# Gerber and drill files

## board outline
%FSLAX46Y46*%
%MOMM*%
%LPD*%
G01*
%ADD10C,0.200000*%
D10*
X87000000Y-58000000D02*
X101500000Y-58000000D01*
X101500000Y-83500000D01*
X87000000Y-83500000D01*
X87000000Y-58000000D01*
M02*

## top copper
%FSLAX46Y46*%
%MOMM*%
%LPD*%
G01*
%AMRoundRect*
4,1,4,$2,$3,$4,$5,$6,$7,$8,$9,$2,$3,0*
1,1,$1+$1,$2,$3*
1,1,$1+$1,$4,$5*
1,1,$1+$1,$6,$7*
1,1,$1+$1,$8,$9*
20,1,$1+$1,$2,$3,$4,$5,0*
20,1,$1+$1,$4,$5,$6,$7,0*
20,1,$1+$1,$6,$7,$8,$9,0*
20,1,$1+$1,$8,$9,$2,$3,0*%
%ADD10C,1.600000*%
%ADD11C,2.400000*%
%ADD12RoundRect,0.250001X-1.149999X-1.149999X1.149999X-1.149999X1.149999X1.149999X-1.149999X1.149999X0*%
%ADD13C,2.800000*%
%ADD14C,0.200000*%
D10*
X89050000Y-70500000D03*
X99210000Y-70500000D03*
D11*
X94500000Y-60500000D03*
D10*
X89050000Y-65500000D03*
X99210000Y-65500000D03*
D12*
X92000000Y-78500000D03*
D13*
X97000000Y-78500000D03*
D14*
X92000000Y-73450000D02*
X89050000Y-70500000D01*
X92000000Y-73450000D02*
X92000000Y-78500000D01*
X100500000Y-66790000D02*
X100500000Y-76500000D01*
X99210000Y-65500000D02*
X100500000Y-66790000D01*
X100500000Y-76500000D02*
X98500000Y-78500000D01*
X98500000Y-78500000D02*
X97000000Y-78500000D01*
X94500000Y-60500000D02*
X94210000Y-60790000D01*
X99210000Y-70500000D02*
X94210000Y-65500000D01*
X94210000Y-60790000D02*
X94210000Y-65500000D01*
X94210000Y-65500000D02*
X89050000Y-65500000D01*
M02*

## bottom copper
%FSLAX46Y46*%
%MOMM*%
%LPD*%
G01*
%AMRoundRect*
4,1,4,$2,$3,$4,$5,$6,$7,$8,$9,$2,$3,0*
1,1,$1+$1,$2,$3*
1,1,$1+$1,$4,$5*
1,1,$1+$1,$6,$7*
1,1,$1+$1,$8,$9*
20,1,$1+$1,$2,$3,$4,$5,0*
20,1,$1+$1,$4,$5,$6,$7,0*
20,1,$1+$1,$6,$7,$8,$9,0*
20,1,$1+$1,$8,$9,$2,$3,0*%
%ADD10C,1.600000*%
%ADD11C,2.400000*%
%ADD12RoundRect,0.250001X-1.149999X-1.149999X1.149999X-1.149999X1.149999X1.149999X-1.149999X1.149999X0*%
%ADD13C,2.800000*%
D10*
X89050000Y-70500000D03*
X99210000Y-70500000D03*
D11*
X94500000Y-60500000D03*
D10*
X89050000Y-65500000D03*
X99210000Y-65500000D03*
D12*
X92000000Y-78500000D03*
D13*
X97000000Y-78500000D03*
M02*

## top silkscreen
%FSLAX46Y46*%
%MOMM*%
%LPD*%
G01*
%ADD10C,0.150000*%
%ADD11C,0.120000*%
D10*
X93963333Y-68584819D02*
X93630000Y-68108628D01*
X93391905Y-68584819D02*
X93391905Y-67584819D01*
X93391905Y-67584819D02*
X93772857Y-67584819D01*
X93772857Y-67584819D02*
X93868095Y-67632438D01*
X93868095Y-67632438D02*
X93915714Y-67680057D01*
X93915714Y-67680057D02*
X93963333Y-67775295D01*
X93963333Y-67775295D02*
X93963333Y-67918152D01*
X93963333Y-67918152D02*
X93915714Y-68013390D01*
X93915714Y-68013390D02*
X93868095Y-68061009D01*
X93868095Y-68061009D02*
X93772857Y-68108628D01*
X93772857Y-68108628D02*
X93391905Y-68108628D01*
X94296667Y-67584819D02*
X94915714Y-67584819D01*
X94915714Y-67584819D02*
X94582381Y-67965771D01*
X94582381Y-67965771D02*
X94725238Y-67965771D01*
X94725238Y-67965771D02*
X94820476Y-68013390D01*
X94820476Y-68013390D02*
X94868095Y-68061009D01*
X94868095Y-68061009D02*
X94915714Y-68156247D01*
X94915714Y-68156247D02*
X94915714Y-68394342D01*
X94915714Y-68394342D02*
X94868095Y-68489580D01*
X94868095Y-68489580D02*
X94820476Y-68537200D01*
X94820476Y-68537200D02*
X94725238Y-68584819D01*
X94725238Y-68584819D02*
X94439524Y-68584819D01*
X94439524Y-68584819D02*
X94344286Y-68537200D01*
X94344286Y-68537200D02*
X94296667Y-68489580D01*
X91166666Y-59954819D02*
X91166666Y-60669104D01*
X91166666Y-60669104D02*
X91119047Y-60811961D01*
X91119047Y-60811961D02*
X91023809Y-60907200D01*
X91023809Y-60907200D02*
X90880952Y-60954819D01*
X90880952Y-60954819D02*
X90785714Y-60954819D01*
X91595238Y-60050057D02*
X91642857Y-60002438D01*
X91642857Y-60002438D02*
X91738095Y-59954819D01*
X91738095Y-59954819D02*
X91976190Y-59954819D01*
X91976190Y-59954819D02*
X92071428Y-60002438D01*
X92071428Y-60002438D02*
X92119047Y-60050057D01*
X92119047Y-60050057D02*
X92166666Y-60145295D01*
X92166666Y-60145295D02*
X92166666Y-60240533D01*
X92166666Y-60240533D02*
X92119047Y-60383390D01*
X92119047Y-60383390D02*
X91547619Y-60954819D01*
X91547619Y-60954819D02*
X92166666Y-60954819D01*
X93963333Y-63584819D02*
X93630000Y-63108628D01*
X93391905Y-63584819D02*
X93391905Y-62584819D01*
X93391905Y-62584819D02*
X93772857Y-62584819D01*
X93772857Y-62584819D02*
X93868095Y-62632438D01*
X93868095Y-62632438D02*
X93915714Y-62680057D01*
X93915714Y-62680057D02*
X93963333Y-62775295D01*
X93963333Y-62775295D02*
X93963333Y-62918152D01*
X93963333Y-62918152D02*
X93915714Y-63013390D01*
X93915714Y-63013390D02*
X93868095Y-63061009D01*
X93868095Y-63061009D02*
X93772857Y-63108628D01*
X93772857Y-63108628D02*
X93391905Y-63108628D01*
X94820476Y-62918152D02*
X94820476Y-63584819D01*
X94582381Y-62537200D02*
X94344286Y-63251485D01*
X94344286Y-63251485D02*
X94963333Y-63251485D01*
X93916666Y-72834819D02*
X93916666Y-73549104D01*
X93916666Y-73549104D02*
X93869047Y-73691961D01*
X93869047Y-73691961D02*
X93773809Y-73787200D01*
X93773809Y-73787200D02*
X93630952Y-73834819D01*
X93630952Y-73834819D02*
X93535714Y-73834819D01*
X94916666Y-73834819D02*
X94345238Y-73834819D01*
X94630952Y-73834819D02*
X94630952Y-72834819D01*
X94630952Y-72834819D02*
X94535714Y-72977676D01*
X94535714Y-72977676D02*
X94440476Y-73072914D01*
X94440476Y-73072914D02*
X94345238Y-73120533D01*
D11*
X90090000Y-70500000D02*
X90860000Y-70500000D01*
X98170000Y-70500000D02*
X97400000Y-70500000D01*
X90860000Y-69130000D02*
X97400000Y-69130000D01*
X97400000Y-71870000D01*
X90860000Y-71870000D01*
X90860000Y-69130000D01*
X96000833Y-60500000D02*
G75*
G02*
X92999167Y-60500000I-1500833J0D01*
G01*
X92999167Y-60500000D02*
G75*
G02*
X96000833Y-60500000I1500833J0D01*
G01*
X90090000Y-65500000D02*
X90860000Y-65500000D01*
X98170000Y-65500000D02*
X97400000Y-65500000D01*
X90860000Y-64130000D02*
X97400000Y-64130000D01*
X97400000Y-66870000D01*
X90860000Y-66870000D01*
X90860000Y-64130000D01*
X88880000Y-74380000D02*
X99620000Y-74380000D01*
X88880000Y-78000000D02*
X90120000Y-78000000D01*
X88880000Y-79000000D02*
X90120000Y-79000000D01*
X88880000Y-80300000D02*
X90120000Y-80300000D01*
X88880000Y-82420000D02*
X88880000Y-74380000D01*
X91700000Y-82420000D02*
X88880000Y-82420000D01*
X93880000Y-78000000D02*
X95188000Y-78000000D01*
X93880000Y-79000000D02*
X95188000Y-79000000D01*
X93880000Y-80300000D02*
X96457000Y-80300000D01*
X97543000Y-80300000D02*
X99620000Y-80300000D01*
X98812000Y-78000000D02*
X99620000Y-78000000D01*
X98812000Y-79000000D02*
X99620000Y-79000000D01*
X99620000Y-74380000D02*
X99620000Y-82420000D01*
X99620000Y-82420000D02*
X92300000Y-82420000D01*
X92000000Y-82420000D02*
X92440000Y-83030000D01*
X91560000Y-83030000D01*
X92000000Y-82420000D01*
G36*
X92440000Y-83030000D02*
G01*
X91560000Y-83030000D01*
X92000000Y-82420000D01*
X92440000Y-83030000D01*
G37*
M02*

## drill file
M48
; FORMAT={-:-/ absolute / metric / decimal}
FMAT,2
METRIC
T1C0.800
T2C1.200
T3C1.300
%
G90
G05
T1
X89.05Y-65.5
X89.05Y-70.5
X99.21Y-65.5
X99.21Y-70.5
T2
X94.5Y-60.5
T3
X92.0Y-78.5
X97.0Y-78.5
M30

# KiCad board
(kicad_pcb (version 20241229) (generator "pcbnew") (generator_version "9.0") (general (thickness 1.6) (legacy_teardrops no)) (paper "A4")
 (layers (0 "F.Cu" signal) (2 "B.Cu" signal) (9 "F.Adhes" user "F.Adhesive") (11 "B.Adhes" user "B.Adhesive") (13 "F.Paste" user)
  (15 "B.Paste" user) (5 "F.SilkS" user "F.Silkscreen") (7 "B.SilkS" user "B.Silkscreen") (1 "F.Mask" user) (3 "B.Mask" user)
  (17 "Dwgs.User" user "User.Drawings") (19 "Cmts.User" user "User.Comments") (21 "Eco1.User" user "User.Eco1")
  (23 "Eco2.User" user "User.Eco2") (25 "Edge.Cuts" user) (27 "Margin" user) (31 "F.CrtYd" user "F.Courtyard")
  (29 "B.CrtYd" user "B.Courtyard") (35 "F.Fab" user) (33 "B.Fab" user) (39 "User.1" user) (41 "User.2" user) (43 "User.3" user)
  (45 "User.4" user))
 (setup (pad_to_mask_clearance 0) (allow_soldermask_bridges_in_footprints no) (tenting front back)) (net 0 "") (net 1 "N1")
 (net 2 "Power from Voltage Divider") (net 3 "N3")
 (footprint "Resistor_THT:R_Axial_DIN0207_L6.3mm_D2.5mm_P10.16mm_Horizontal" (layer "F.Cu") (at 89.05 70.5)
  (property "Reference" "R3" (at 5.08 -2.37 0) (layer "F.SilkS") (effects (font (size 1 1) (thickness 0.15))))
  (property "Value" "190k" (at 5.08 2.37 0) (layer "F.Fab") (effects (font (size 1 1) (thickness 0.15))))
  (fp_line (start 1.04 0) (end 1.81 0) (stroke (width 0.12) (type solid)) (layer "F.SilkS"))
  (fp_line (start 9.12 0) (end 8.35 0) (stroke (width 0.12) (type solid)) (layer "F.SilkS"))
  (fp_rect (start 1.81 -1.37) (end 8.35 1.37) (stroke (width 0.12) (type solid)) (fill no) (layer "F.SilkS"))
  (pad "1" thru_hole circle (at 0 0) (size 1.6 1.6) (drill 0.8) (layers "*.Cu" "*.Mask") (remove_unused_layers no) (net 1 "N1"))
  (pad "2" thru_hole circle (at 10.16 0) (size 1.6 1.6) (drill 0.8) (layers "*.Cu" "*.Mask") (remove_unused_layers no)
   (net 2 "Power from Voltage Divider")))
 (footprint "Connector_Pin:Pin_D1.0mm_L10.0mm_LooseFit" (layer "F.Cu") (at 94.5 60.5)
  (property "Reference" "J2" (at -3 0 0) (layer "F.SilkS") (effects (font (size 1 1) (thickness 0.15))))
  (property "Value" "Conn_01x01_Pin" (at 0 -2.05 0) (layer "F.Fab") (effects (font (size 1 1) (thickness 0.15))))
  (fp_circle (center 0 0) (end 1.5 0.05) (stroke (width 0.12) (type solid)) (fill no) (layer "F.SilkS"))
  (pad "1" thru_hole circle (at 0 0) (size 2.4 2.4) (drill 1.2) (layers "*.Cu" "*.Mask") (remove_unused_layers no)
   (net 2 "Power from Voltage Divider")))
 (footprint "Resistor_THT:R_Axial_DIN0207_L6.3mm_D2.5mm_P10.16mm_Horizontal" (layer "F.Cu") (at 89.05 65.5)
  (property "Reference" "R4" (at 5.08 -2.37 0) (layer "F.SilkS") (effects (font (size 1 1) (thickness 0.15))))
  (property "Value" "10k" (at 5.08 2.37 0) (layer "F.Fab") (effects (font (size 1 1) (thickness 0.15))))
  (fp_line (start 1.04 0) (end 1.81 0) (stroke (width 0.12) (type solid)) (layer "F.SilkS"))
  (fp_line (start 9.12 0) (end 8.35 0) (stroke (width 0.12) (type solid)) (layer "F.SilkS"))
  (fp_rect (start 1.81 -1.37) (end 8.35 1.37) (stroke (width 0.12) (type solid)) (fill no) (layer "F.SilkS"))
  (pad "1" thru_hole circle (at 0 0) (size 1.6 1.6) (drill 0.8) (layers "*.Cu" "*.Mask") (remove_unused_layers no)
   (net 2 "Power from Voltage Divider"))
  (pad "2" thru_hole circle (at 10.16 0) (size 1.6 1.6) (drill 0.8) (layers "*.Cu" "*.Mask") (remove_unused_layers no) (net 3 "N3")))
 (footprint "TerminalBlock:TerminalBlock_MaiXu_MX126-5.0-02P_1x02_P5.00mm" (layer "F.Cu") (at 92 78.5)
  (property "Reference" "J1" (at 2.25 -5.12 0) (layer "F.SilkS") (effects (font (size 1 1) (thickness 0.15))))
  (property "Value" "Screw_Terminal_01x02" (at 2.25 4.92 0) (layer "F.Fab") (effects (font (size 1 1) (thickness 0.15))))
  (fp_line (start -3.12 -4.12) (end 7.62 -4.12) (stroke (width 0.12) (type solid)) (layer "F.SilkS"))
  (fp_line (start -3.12 -0.5) (end -1.88 -0.5) (stroke (width 0.12) (type solid)) (layer "F.SilkS"))
  (fp_line (start -3.12 0.5) (end -1.88 0.5) (stroke (width 0.12) (type solid)) (layer "F.SilkS"))
  (fp_line (start -3.12 1.8) (end -1.88 1.8) (stroke (width 0.12) (type solid)) (layer "F.SilkS"))
  (fp_line (start -3.12 3.92) (end -3.12 -4.12) (stroke (width 0.12) (type solid)) (layer "F.SilkS"))
  (fp_line (start -0.3 3.92) (end -3.12 3.92) (stroke (width 0.12) (type solid)) (layer "F.SilkS"))
  (fp_line (start 1.88 -0.5) (end 3.188 -0.5) (stroke (width 0.12) (type solid)) (layer "F.SilkS"))
  (fp_line (start 1.88 0.5) (end 3.188 0.5) (stroke (width 0.12) (type solid)) (layer "F.SilkS"))
  (fp_line (start 1.88 1.8) (end 4.457 1.8) (stroke (width 0.12) (type solid)) (layer "F.SilkS"))
  (fp_line (start 5.543 1.8) (end 7.62 1.8) (stroke (width 0.12) (type solid)) (layer "F.SilkS"))
  (fp_line (start 6.812 -0.5) (end 7.62 -0.5) (stroke (width 0.12) (type solid)) (layer "F.SilkS"))
  (fp_line (start 6.812 0.5) (end 7.62 0.5) (stroke (width 0.12) (type solid)) (layer "F.SilkS"))
  (fp_line (start 7.62 -4.12) (end 7.62 3.92) (stroke (width 0.12) (type solid)) (layer "F.SilkS"))
  (fp_line (start 7.62 3.92) (end 0.3 3.92) (stroke (width 0.12) (type solid)) (layer "F.SilkS"))
  (fp_poly (pts (xy 0 3.92) (xy 0.44 4.53) (xy -0.44 4.53)) (stroke (width 0.12) (type solid)) (fill yes) (layer "F.SilkS"))
  (pad "1" thru_hole roundrect (at 0 0) (size 2.8 2.8) (drill 1.3) (layers "*.Cu" "*.Mask") (remove_unused_layers no)
   (roundrect_rratio 0.089286) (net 1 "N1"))
  (pad "2" thru_hole circle (at 5 0) (size 2.8 2.8) (drill 1.3) (layers "*.Cu" "*.Mask") (remove_unused_layers no) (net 3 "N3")))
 (gr_rect (start 87 58) (end 101.5 83.5) (stroke (width 0.2) (type solid)) (fill no) (layer "Edge.Cuts"))
 (segment (start 92 73.45) (end 89.05 70.5) (width 0.2) (layer "F.Cu") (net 1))
 (segment (start 92 73.45) (end 92 78.5) (width 0.2) (layer "F.Cu") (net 1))
 (segment (start 100.5 66.79) (end 100.5 76.5) (width 0.2) (layer "F.Cu") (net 3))
 (segment (start 99.21 65.5) (end 100.5 66.79) (width 0.2) (layer "F.Cu") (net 3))
 (segment (start 100.5 76.5) (end 98.5 78.5) (width 0.2) (layer "F.Cu") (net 3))
 (segment (start 98.5 78.5) (end 97 78.5) (width 0.2) (layer "F.Cu") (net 3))
 (segment (start 94.5 60.5) (end 94.21 60.79) (width 0.2) (layer "F.Cu") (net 2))
 (segment (start 99.21 70.5) (end 94.21 65.5) (width 0.2) (layer "F.Cu") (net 2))
 (segment (start 94.21 60.79) (end 94.21 65.5) (width 0.2) (layer "F.Cu") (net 2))
 (segment (start 94.21 65.5) (end 89.05 65.5) (width 0.2) (layer "F.Cu") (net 2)))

